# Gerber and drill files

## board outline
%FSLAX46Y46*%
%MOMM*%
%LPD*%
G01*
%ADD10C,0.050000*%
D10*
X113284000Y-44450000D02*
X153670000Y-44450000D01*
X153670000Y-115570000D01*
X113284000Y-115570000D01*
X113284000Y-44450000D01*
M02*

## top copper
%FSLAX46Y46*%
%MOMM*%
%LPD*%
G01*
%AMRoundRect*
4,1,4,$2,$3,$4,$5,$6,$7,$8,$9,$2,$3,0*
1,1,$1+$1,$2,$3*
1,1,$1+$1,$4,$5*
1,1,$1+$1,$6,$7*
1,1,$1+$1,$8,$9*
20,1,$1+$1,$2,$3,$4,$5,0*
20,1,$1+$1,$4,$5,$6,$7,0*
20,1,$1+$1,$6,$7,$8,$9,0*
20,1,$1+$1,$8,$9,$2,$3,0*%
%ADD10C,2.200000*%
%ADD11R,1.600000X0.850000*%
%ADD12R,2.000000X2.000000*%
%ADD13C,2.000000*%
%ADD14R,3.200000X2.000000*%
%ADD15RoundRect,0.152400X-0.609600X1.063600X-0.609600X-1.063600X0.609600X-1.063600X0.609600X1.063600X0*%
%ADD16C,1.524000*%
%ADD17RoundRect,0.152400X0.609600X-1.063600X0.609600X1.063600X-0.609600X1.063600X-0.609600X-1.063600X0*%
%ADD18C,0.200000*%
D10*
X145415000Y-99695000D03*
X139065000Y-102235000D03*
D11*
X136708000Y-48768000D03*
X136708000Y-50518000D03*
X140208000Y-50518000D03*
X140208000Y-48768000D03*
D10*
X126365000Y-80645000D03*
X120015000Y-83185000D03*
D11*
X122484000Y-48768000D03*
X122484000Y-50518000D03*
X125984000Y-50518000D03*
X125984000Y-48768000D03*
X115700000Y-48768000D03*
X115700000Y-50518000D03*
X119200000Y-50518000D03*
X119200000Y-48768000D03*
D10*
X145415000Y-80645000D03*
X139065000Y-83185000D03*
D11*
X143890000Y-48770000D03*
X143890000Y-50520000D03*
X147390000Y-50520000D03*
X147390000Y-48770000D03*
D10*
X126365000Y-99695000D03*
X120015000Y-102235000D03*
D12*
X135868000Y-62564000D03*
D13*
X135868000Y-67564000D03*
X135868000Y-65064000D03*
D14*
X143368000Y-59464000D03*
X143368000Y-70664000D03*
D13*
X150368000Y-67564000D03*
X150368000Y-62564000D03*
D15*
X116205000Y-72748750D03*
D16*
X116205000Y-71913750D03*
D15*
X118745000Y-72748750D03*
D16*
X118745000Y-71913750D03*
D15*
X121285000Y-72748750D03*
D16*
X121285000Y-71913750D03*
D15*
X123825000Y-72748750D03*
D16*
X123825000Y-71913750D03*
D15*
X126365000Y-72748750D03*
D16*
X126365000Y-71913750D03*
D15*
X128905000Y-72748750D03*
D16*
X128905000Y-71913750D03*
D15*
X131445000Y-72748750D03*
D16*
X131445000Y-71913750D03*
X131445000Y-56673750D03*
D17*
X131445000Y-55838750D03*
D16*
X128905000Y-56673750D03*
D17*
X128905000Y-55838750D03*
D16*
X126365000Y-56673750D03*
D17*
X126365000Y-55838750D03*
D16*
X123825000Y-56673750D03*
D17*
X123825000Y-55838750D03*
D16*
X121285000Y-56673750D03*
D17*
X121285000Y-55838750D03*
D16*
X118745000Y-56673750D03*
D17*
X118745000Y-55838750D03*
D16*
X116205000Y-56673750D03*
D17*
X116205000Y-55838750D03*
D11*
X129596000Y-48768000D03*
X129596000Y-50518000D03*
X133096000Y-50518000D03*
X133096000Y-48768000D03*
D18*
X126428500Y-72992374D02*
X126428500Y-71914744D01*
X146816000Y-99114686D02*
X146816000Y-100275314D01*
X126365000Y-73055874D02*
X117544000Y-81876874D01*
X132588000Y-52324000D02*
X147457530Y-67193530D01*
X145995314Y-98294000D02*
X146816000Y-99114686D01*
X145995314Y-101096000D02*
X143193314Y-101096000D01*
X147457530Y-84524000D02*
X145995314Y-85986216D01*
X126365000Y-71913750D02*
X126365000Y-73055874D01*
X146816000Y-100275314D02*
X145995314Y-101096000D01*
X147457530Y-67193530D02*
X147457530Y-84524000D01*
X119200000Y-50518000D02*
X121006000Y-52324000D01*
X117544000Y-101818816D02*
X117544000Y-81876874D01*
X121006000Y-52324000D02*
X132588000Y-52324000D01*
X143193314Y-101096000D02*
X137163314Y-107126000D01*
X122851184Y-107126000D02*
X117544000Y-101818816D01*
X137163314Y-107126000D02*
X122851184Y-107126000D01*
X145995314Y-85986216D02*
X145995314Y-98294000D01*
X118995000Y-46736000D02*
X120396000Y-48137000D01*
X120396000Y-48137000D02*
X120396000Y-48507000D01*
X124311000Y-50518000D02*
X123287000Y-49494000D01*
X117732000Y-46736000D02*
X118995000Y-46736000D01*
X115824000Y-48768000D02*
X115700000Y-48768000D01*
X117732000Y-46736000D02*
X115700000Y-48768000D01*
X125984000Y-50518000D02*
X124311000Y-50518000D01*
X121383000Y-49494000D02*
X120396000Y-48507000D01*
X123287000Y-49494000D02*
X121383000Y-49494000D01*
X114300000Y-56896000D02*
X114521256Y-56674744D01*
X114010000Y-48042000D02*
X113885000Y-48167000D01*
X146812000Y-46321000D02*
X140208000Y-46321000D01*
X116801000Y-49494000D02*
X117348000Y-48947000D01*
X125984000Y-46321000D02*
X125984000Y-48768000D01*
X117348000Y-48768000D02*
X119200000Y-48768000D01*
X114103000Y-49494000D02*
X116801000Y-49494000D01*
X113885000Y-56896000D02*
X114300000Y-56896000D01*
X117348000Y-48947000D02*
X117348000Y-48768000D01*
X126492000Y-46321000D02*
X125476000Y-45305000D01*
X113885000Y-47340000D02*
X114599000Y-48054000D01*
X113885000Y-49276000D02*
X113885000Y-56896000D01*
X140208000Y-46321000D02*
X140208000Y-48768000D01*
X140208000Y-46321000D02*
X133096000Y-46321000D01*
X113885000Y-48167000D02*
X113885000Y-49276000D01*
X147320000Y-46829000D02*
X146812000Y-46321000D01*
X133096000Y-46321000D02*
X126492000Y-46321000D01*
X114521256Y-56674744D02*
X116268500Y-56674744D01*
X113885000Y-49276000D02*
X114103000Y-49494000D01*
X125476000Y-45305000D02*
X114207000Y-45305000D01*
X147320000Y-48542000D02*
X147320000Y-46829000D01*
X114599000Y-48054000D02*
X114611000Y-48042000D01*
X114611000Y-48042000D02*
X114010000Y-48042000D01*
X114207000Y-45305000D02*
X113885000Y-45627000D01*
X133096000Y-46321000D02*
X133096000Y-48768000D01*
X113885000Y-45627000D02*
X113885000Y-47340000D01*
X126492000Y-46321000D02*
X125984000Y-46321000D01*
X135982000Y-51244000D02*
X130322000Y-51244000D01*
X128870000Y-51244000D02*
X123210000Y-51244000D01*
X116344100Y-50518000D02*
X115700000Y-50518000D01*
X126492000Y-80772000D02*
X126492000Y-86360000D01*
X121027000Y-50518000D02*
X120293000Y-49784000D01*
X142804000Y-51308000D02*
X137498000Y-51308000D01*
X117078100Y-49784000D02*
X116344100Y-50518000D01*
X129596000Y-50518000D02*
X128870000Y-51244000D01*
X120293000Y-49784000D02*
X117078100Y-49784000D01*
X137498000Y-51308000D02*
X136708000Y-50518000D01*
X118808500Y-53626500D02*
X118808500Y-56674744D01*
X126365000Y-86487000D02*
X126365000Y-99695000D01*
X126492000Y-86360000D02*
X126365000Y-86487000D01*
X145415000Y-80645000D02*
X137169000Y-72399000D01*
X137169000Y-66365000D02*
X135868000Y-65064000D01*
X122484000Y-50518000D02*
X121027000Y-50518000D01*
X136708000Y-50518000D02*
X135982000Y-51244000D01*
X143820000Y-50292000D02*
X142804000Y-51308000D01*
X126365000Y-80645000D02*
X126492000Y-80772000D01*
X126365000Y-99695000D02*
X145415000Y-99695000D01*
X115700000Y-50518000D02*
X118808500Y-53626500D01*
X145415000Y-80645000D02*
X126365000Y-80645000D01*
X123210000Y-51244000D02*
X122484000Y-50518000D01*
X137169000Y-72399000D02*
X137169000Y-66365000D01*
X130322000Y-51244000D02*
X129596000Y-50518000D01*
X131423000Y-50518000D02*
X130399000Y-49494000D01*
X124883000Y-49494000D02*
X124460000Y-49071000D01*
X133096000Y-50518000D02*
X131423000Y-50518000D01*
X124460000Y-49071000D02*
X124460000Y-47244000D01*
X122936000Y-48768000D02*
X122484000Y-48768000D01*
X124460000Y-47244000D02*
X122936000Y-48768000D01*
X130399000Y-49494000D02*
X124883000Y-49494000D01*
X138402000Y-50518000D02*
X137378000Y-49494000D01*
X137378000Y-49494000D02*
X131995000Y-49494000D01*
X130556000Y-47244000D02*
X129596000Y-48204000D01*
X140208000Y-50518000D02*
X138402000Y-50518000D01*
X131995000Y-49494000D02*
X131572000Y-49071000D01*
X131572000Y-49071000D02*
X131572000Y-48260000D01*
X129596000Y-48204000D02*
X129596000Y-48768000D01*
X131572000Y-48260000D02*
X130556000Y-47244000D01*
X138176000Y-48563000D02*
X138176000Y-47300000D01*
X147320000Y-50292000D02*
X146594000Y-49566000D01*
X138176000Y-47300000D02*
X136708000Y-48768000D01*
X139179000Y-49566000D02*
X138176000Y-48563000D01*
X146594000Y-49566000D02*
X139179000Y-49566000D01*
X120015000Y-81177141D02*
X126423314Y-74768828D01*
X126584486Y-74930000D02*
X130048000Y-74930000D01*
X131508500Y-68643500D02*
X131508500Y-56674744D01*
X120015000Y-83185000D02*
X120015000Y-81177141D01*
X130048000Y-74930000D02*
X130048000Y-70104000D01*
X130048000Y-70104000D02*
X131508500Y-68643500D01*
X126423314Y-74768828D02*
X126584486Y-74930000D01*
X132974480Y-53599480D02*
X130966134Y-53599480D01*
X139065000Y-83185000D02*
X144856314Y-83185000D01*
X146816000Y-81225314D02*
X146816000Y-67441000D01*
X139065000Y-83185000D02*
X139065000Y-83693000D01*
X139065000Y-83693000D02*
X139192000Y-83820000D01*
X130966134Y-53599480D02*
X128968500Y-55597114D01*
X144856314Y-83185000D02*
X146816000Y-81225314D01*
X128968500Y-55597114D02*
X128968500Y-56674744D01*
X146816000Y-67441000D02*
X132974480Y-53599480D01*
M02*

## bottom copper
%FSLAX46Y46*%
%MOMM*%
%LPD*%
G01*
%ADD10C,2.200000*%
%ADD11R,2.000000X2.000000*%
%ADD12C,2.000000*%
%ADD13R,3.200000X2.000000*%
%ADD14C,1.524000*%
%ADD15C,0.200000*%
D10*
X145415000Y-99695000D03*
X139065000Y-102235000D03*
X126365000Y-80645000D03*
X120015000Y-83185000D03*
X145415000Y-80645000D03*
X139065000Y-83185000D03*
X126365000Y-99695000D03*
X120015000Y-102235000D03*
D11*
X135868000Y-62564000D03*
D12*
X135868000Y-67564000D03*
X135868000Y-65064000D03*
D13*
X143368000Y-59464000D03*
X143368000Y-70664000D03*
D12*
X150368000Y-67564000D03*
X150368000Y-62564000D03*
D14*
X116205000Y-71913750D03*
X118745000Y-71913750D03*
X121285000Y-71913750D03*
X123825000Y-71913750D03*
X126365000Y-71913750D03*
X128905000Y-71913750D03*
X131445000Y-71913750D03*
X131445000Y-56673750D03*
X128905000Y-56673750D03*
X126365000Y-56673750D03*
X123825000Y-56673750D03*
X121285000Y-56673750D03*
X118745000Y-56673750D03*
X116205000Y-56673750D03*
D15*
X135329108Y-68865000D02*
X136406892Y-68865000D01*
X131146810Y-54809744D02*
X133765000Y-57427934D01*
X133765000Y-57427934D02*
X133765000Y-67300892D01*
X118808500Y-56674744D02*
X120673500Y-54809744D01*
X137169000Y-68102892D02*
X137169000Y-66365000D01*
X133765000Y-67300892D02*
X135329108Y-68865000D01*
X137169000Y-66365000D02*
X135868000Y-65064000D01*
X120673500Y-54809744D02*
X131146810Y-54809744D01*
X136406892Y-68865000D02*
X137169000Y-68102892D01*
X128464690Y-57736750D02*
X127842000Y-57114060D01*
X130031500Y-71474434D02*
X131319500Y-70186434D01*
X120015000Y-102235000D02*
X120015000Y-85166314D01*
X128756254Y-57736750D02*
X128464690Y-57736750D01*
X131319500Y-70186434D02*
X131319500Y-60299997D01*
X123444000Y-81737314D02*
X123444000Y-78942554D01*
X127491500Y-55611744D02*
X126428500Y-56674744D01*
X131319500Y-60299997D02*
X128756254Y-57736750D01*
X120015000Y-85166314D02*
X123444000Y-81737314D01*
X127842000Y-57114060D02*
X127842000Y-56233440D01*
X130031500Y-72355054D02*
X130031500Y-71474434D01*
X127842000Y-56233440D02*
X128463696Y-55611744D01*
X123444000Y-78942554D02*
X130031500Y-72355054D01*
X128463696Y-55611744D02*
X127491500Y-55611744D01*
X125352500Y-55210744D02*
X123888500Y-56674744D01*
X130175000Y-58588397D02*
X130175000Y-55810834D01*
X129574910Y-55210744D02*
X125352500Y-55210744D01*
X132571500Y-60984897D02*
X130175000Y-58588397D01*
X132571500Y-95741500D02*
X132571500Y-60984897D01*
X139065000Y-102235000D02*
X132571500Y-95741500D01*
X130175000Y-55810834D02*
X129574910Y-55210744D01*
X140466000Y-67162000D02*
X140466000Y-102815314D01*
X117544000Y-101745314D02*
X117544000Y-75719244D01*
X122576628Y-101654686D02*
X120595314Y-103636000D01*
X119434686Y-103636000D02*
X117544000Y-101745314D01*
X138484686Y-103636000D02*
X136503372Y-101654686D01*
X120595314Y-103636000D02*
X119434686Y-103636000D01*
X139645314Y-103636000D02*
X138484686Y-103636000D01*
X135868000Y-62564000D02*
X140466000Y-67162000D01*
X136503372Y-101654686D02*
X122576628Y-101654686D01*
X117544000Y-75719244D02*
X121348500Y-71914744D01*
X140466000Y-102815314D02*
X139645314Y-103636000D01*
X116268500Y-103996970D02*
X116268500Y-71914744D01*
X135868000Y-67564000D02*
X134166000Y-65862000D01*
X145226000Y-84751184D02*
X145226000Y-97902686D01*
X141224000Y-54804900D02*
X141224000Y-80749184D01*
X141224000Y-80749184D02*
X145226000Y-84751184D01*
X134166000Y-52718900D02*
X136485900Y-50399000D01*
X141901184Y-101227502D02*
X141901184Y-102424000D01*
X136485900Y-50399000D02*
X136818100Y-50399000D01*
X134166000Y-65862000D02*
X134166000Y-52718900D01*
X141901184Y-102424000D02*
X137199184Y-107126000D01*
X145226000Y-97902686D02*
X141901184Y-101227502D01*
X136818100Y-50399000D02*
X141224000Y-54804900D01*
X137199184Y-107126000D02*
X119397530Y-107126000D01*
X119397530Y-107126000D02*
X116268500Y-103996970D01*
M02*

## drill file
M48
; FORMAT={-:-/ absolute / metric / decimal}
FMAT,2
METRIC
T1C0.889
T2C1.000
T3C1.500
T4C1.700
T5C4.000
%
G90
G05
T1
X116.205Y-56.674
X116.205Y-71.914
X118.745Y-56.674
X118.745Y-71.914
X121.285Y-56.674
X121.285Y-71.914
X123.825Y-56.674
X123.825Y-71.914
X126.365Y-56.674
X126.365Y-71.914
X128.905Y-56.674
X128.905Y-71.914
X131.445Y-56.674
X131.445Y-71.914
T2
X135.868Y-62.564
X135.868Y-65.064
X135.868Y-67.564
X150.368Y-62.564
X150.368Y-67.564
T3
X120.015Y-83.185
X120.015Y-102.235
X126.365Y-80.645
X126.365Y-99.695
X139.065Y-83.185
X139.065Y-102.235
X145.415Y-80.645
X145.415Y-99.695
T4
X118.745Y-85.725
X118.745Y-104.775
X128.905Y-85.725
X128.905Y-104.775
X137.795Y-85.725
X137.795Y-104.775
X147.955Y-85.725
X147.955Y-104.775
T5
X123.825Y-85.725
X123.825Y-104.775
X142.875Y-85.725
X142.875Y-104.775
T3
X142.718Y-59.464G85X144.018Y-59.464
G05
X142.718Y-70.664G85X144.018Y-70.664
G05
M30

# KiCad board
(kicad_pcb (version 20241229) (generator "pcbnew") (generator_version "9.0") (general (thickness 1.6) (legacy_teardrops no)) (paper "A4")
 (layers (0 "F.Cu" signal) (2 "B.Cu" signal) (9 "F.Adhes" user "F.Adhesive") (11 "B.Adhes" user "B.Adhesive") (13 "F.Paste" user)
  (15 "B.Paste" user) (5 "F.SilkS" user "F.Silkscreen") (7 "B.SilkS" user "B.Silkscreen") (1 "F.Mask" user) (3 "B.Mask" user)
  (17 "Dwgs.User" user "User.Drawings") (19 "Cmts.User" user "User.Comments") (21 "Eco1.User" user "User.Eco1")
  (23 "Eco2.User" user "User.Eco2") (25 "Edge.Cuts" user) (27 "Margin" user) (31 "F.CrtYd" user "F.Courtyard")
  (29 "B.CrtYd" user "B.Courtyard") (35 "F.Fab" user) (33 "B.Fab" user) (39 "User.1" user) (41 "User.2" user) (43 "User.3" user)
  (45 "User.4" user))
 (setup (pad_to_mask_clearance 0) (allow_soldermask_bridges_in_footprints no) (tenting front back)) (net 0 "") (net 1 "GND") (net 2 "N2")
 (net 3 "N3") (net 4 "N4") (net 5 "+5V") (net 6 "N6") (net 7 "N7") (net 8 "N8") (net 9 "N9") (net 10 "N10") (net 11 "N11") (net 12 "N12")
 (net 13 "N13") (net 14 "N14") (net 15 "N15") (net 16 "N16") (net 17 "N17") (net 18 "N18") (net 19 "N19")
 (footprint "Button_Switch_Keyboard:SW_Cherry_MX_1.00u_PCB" (layer "F.Cu") (at 145.415 99.695)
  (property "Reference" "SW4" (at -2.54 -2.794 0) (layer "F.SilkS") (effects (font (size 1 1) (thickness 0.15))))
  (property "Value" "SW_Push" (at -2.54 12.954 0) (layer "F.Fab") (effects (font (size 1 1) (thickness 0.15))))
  (pad "" np_thru_hole circle (at -7.62 5.08) (size 1.7 1.7) (drill 1.7) (layers "*.Cu" "*.Mask"))
  (pad "" np_thru_hole circle (at -2.54 5.08) (size 4 4) (drill 4) (layers "*.Cu" "*.Mask"))
  (pad "" np_thru_hole circle (at 2.54 5.08) (size 1.7 1.7) (drill 1.7) (layers "*.Cu" "*.Mask"))
  (pad "1" thru_hole circle (at 0 0) (size 2.2 2.2) (drill 1.5) (layers "*.Cu" "*.Mask") (remove_unused_layers no) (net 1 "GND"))
  (pad "2" thru_hole circle (at -6.35 2.54) (size 2.2 2.2) (drill 1.5) (layers "*.Cu" "*.Mask") (remove_unused_layers no) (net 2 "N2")))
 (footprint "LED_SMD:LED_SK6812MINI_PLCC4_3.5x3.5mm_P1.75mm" (layer "F.Cu") (at 138.458 49.643)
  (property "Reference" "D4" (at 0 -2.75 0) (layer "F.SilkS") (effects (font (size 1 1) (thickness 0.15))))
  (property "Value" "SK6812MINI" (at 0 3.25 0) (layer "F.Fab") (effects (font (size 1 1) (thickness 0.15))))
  (pad "1" smd rect (at -1.75 -0.875) (size 1.6 0.85) (layers "F.Cu" "F.Mask" "F.Paste") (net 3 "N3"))
  (pad "2" smd rect (at -1.75 0.875) (size 1.6 0.85) (layers "F.Cu" "F.Mask" "F.Paste") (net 1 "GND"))
  (pad "3" smd rect (at 1.75 0.875) (size 1.6 0.85) (layers "F.Cu" "F.Mask" "F.Paste") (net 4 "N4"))
  (pad "4" smd rect (at 1.75 -0.875) (size 1.6 0.85) (layers "F.Cu" "F.Mask" "F.Paste") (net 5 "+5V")))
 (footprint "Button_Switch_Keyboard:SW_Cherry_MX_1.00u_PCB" (layer "F.Cu") (at 126.365 80.645)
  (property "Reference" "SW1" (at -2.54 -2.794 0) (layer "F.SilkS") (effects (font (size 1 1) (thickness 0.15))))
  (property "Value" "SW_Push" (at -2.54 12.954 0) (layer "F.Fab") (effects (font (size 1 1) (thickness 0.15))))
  (pad "" np_thru_hole circle (at -7.62 5.08) (size 1.7 1.7) (drill 1.7) (layers "*.Cu" "*.Mask"))
  (pad "" np_thru_hole circle (at -2.54 5.08) (size 4 4) (drill 4) (layers "*.Cu" "*.Mask"))
  (pad "" np_thru_hole circle (at 2.54 5.08) (size 1.7 1.7) (drill 1.7) (layers "*.Cu" "*.Mask"))
  (pad "1" thru_hole circle (at 0 0) (size 2.2 2.2) (drill 1.5) (layers "*.Cu" "*.Mask") (remove_unused_layers no) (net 1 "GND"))
  (pad "2" thru_hole circle (at -6.35 2.54) (size 2.2 2.2) (drill 1.5) (layers "*.Cu" "*.Mask") (remove_unused_layers no) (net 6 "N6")))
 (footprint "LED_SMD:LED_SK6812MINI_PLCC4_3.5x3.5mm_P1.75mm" (layer "F.Cu") (at 124.234 49.643)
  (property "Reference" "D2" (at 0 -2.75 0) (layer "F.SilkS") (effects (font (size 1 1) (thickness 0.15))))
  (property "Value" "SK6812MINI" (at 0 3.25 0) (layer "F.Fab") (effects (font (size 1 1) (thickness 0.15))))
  (pad "1" smd rect (at -1.75 -0.875) (size 1.6 0.85) (layers "F.Cu" "F.Mask" "F.Paste") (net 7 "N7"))
  (pad "2" smd rect (at -1.75 0.875) (size 1.6 0.85) (layers "F.Cu" "F.Mask" "F.Paste") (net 1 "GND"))
  (pad "3" smd rect (at 1.75 0.875) (size 1.6 0.85) (layers "F.Cu" "F.Mask" "F.Paste") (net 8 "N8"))
  (pad "4" smd rect (at 1.75 -0.875) (size 1.6 0.85) (layers "F.Cu" "F.Mask" "F.Paste") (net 5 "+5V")))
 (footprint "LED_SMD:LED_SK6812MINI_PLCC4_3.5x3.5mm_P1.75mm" (layer "F.Cu") (at 117.45 49.643)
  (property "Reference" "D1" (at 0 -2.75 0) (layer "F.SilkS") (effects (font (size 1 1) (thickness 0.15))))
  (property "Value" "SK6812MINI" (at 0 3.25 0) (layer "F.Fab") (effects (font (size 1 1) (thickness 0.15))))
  (pad "1" smd rect (at -1.75 -0.875) (size 1.6 0.85) (layers "F.Cu" "F.Mask" "F.Paste") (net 8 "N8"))
  (pad "2" smd rect (at -1.75 0.875) (size 1.6 0.85) (layers "F.Cu" "F.Mask" "F.Paste") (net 1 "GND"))
  (pad "3" smd rect (at 1.75 0.875) (size 1.6 0.85) (layers "F.Cu" "F.Mask" "F.Paste") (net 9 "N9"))
  (pad "4" smd rect (at 1.75 -0.875) (size 1.6 0.85) (layers "F.Cu" "F.Mask" "F.Paste") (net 5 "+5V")))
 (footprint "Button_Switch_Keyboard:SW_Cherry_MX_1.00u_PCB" (layer "F.Cu") (at 145.415 80.645)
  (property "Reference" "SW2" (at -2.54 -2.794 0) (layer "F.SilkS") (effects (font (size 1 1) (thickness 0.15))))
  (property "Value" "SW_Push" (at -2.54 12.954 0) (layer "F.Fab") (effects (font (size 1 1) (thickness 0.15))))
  (pad "" np_thru_hole circle (at -7.62 5.08) (size 1.7 1.7) (drill 1.7) (layers "*.Cu" "*.Mask"))
  (pad "" np_thru_hole circle (at -2.54 5.08) (size 4 4) (drill 4) (layers "*.Cu" "*.Mask"))
  (pad "" np_thru_hole circle (at 2.54 5.08) (size 1.7 1.7) (drill 1.7) (layers "*.Cu" "*.Mask"))
  (pad "1" thru_hole circle (at 0 0) (size 2.2 2.2) (drill 1.5) (layers "*.Cu" "*.Mask") (remove_unused_layers no) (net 1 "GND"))
  (pad "2" thru_hole circle (at -6.35 2.54) (size 2.2 2.2) (drill 1.5) (layers "*.Cu" "*.Mask") (remove_unused_layers no) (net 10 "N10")))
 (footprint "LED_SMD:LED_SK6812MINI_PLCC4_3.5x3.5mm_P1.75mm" (layer "F.Cu") (at 145.64 49.645)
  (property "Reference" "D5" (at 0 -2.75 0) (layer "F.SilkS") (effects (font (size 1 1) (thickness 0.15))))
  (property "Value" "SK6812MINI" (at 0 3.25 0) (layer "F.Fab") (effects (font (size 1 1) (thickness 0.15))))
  (pad "1" smd rect (at -1.75 -0.875) (size 1.6 0.85) (layers "F.Cu" "F.Mask" "F.Paste") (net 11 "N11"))
  (pad "2" smd rect (at -1.75 0.875) (size 1.6 0.85) (layers "F.Cu" "F.Mask" "F.Paste") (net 1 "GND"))
  (pad "3" smd rect (at 1.75 0.875) (size 1.6 0.85) (layers "F.Cu" "F.Mask" "F.Paste") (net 3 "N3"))
  (pad "4" smd rect (at 1.75 -0.875) (size 1.6 0.85) (layers "F.Cu" "F.Mask" "F.Paste") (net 5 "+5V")))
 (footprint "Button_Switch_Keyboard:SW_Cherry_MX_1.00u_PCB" (layer "F.Cu") (at 126.365 99.695)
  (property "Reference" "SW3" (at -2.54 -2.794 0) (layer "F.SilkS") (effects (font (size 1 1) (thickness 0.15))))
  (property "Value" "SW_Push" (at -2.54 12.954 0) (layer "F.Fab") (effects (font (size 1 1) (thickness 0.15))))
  (pad "" np_thru_hole circle (at -7.62 5.08) (size 1.7 1.7) (drill 1.7) (layers "*.Cu" "*.Mask"))
  (pad "" np_thru_hole circle (at -2.54 5.08) (size 4 4) (drill 4) (layers "*.Cu" "*.Mask"))
  (pad "" np_thru_hole circle (at 2.54 5.08) (size 1.7 1.7) (drill 1.7) (layers "*.Cu" "*.Mask"))
  (pad "1" thru_hole circle (at 0 0) (size 2.2 2.2) (drill 1.5) (layers "*.Cu" "*.Mask") (remove_unused_layers no) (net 1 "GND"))
  (pad "2" thru_hole circle (at -6.35 2.54) (size 2.2 2.2) (drill 1.5) (layers "*.Cu" "*.Mask") (remove_unused_layers no) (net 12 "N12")))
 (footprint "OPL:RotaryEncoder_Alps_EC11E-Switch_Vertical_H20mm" (layer "F.Cu") (at 135.868 62.564)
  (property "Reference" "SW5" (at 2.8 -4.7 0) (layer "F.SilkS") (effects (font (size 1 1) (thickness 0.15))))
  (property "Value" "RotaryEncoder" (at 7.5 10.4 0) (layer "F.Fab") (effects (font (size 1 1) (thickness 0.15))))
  (pad "A" thru_hole rect (at 0 0) (size 2 2) (drill 1) (layers "*.Cu" "*.Mask") (remove_unused_layers no) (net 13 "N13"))
  (pad "B" thru_hole circle (at 0 5) (size 2 2) (drill 1) (layers "*.Cu" "*.Mask") (remove_unused_layers no) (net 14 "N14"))
  (pad "C" thru_hole circle (at 0 2.5) (size 2 2) (drill 1) (layers "*.Cu" "*.Mask") (remove_unused_layers no) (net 1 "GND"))
  (pad "MP" thru_hole rect (at 7.5 -3.1) (size 3.2 2) (drill oval 2.8 1.5) (layers "*.Cu" "*.Mask") (remove_unused_layers no))
  (pad "MP" thru_hole rect (at 7.5 8.1) (size 3.2 2) (drill oval 2.8 1.5) (layers "*.Cu" "*.Mask") (remove_unused_layers no))
  (pad "S1" thru_hole circle (at 14.5 5) (size 2 2) (drill 1) (layers "*.Cu" "*.Mask") (remove_unused_layers no))
  (pad "S2" thru_hole circle (at 14.5 0) (size 2 2) (drill 1) (layers "*.Cu" "*.Mask") (remove_unused_layers no)))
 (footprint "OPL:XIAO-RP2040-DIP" (layer "F.Cu") (at 123.825 64.29375 90)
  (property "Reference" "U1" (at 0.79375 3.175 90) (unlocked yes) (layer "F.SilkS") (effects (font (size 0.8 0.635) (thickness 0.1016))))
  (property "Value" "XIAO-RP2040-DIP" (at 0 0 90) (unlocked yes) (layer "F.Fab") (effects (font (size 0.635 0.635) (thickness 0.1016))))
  (pad "1" smd roundrect (at -8.455 -7.62 270) (size 2.432 1.524) (layers "F.Cu" "F.Mask") (roundrect_rratio 0.1) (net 14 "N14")
   (thermal_bridge_angle 45))
  (pad "1" thru_hole circle (at -7.62 -7.62 270) (size 1.524 1.524) (drill 0.889) (layers "*.Cu" "*.Mask") (remove_unused_layers no)
   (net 14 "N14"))
  (pad "2" smd roundrect (at -8.455 -5.08 270) (size 2.432 1.524) (layers "F.Cu" "F.Mask") (roundrect_rratio 0.1) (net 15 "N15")
   (thermal_bridge_angle 45))
  (pad "2" thru_hole circle (at -7.62 -5.08 270) (size 1.524 1.524) (drill 0.889) (layers "*.Cu" "*.Mask") (remove_unused_layers no)
   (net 15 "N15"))
  (pad "3" smd roundrect (at -8.455 -2.54 270) (size 2.432 1.524) (layers "F.Cu" "F.Mask") (roundrect_rratio 0.1) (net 13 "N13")
   (thermal_bridge_angle 45))
  (pad "3" thru_hole circle (at -7.62 -2.54 270) (size 1.524 1.524) (drill 0.889) (layers "*.Cu" "*.Mask") (remove_unused_layers no)
   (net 13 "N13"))
  (pad "4" smd roundrect (at -8.455 0 270) (size 2.432 1.524) (layers "F.Cu" "F.Mask") (roundrect_rratio 0.1) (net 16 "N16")
   (thermal_bridge_angle 45))
  (pad "4" thru_hole circle (at -7.62 0 270) (size 1.524 1.524) (drill 0.889) (layers "*.Cu" "*.Mask") (remove_unused_layers no)
   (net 16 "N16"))
  (pad "5" smd roundrect (at -8.455 2.54 270) (size 2.432 1.524) (layers "F.Cu" "F.Mask") (roundrect_rratio 0.1) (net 9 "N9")
   (thermal_bridge_angle 45))
  (pad "5" thru_hole circle (at -7.62 2.54 270) (size 1.524 1.524) (drill 0.889) (layers "*.Cu" "*.Mask") (remove_unused_layers no)
   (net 9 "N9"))
  (pad "6" smd roundrect (at -8.455 5.08 270) (size 2.432 1.524) (layers "F.Cu" "F.Mask") (roundrect_rratio 0.1) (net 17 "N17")
   (thermal_bridge_angle 45))
  (pad "6" thru_hole circle (at -7.62 5.08 270) (size 1.524 1.524) (drill 0.889) (layers "*.Cu" "*.Mask") (remove_unused_layers no)
   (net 17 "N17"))
  (pad "7" smd roundrect (at -8.455 7.62 270) (size 2.432 1.524) (layers "F.Cu" "F.Mask") (roundrect_rratio 0.1) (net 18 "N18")
   (thermal_bridge_angle 45))
  (pad "7" thru_hole circle (at -7.62 7.62 270) (size 1.524 1.524) (drill 0.889) (layers "*.Cu" "*.Mask") (remove_unused_layers no)
   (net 18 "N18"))
  (pad "8" thru_hole circle (at 7.62 7.62 90) (size 1.524 1.524) (drill 0.889) (layers "*.Cu" "*.Mask") (remove_unused_layers no)
   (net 6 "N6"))
  (pad "8" smd roundrect (at 8.455 7.62 90) (size 2.432 1.524) (layers "F.Cu" "F.Mask") (roundrect_rratio 0.1) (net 6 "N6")
   (thermal_bridge_angle 45))
  (pad "9" thru_hole circle (at 7.62 5.08 90) (size 1.524 1.524) (drill 0.889) (layers "*.Cu" "*.Mask") (remove_unused_layers no)
   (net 10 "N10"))
  (pad "9" smd roundrect (at 8.455 5.08 90) (size 2.432 1.524) (layers "F.Cu" "F.Mask") (roundrect_rratio 0.1) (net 10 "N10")
   (thermal_bridge_angle 45))
  (pad "10" thru_hole circle (at 7.62 2.54 90) (size 1.524 1.524) (drill 0.889) (layers "*.Cu" "*.Mask") (remove_unused_layers no)
   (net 12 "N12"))
  (pad "10" smd roundrect (at 8.455 2.54 90) (size 2.432 1.524) (layers "F.Cu" "F.Mask") (roundrect_rratio 0.1) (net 12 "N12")
   (thermal_bridge_angle 45))
  (pad "11" thru_hole circle (at 7.62 0 90) (size 1.524 1.524) (drill 0.889) (layers "*.Cu" "*.Mask") (remove_unused_layers no) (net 2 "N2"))
  (pad "11" smd roundrect (at 8.455 0 90) (size 2.432 1.524) (layers "F.Cu" "F.Mask") (roundrect_rratio 0.1) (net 2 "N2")
   (thermal_bridge_angle 45))
  (pad "12" thru_hole circle (at 7.62 -2.54 90) (size 1.524 1.524) (drill 0.889) (layers "*.Cu" "*.Mask") (remove_unused_layers no)
   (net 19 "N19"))
  (pad "12" smd roundrect (at 8.455 -2.54 90) (size 2.432 1.524) (layers "F.Cu" "F.Mask") (roundrect_rratio 0.1) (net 19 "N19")
   (thermal_bridge_angle 45))
  (pad "13" thru_hole circle (at 7.62 -5.08 90) (size 1.524 1.524) (drill 0.889) (layers "*.Cu" "*.Mask") (remove_unused_layers no)
   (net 1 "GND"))
  (pad "13" smd roundrect (at 8.455 -5.08 90) (size 2.432 1.524) (layers "F.Cu" "F.Mask") (roundrect_rratio 0.1) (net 1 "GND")
   (thermal_bridge_angle 45))
  (pad "14" thru_hole circle (at 7.62 -7.62 90) (size 1.524 1.524) (drill 0.889) (layers "*.Cu" "*.Mask") (remove_unused_layers no)
   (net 5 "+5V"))
  (pad "14" smd roundrect (at 8.455 -7.62 90) (size 2.432 1.524) (layers "F.Cu" "F.Mask") (roundrect_rratio 0.1) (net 5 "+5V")
   (thermal_bridge_angle 45)))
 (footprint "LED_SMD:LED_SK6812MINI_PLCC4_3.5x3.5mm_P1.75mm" (layer "F.Cu") (at 131.346 49.643)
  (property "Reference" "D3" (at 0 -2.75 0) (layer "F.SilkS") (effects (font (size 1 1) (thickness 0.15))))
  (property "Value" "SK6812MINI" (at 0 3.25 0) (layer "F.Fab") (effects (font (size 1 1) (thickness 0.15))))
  (pad "1" smd rect (at -1.75 -0.875) (size 1.6 0.85) (layers "F.Cu" "F.Mask" "F.Paste") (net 4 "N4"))
  (pad "2" smd rect (at -1.75 0.875) (size 1.6 0.85) (layers "F.Cu" "F.Mask" "F.Paste") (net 1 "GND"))
  (pad "3" smd rect (at 1.75 0.875) (size 1.6 0.85) (layers "F.Cu" "F.Mask" "F.Paste") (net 7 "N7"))
  (pad "4" smd rect (at 1.75 -0.875) (size 1.6 0.85) (layers "F.Cu" "F.Mask" "F.Paste") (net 5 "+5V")))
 (gr_rect (start 113.284 44.45) (end 153.67 115.57) (stroke (width 0.05) (type default)) (fill no) (layer "Edge.Cuts"))
 (segment (start 126.4285 72.992374) (end 126.4285 71.914744) (width 0.2) (layer "F.Cu") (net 9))
 (segment (start 146.816 99.114686) (end 146.816 100.275314) (width 0.2) (layer "F.Cu") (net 9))
 (segment (start 126.365 73.055874) (end 117.544 81.876874) (width 0.2) (layer "F.Cu") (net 9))
 (segment (start 132.588 52.324) (end 147.45753 67.19353) (width 0.2) (layer "F.Cu") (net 9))
 (segment (start 145.995314 98.294) (end 146.816 99.114686) (width 0.2) (layer "F.Cu") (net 9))
 (segment (start 145.995314 101.096) (end 143.193314 101.096) (width 0.2) (layer "F.Cu") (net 9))
 (segment (start 147.45753 84.524) (end 145.995314 85.986216) (width 0.2) (layer "F.Cu") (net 9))
 (segment (start 126.365 71.91375) (end 126.365 73.055874) (width 0.2) (layer "F.Cu") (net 9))
 (segment (start 146.816 100.275314) (end 145.995314 101.096) (width 0.2) (layer "F.Cu") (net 9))
 (segment (start 147.45753 67.19353) (end 147.45753 84.524) (width 0.2) (layer "F.Cu") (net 9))
 (segment (start 119.2 50.518) (end 121.006 52.324) (width 0.2) (layer "F.Cu") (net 9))
 (segment (start 117.544 101.818816) (end 117.544 81.876874) (width 0.2) (layer "F.Cu") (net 9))
 (segment (start 121.006 52.324) (end 132.588 52.324) (width 0.2) (layer "F.Cu") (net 9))
 (segment (start 143.193314 101.096) (end 137.163314 107.126) (width 0.2) (layer "F.Cu") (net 9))
 (segment (start 122.851184 107.126) (end 117.544 101.818816) (width 0.2) (layer "F.Cu") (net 9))
 (segment (start 137.163314 107.126) (end 122.851184 107.126) (width 0.2) (layer "F.Cu") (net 9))
 (segment (start 145.995314 85.986216) (end 145.995314 98.294) (width 0.2) (layer "F.Cu") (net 9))
 (segment (start 118.995 46.736) (end 120.396 48.137) (width 0.2) (layer "F.Cu") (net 8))
 (segment (start 120.396 48.137) (end 120.396 48.507) (width 0.2) (layer "F.Cu") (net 8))
 (segment (start 124.311 50.518) (end 123.287 49.494) (width 0.2) (layer "F.Cu") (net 8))
 (segment (start 117.732 46.736) (end 118.995 46.736) (width 0.2) (layer "F.Cu") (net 8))
 (segment (start 115.824 48.768) (end 115.7 48.768) (width 0.2) (layer "F.Cu") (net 8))
 (segment (start 117.732 46.736) (end 115.7 48.768) (width 0.2) (layer "F.Cu") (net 8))
 (segment (start 125.984 50.518) (end 124.311 50.518) (width 0.2) (layer "F.Cu") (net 8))
 (segment (start 121.383 49.494) (end 120.396 48.507) (width 0.2) (layer "F.Cu") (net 8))
 (segment (start 123.287 49.494) (end 121.383 49.494) (width 0.2) (layer "F.Cu") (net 8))
 (segment (start 114.3 56.896) (end 114.521256 56.674744) (width 0.2) (layer "F.Cu") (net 5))
 (segment (start 114.01 48.042) (end 113.885 48.167) (width 0.2) (layer "F.Cu") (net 5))
 (segment (start 146.812 46.321) (end 140.208 46.321) (width 0.2) (layer "F.Cu") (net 5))
 (segment (start 116.801 49.494) (end 117.348 48.947) (width 0.2) (layer "F.Cu") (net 5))
 (segment (start 125.984 46.321) (end 125.984 48.768) (width 0.2) (layer "F.Cu") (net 5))
 (segment (start 117.348 48.768) (end 119.2 48.768) (width 0.2) (layer "F.Cu") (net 5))
 (segment (start 114.103 49.494) (end 116.801 49.494) (width 0.2) (layer "F.Cu") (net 5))
 (segment (start 113.885 56.896) (end 114.3 56.896) (width 0.2) (layer "F.Cu") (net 5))
 (segment (start 117.348 48.947) (end 117.348 48.768) (width 0.2) (layer "F.Cu") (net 5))
 (segment (start 126.492 46.321) (end 125.476 45.305) (width 0.2) (layer "F.Cu") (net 5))
 (segment (start 113.885 47.34) (end 114.599 48.054) (width 0.2) (layer "F.Cu") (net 5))
 (segment (start 113.885 49.276) (end 113.885 56.896) (width 0.2) (layer "F.Cu") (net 5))
 (segment (start 140.208 46.321) (end 140.208 48.768) (width 0.2) (layer "F.Cu") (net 5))
 (segment (start 140.208 46.321) (end 133.096 46.321) (width 0.2) (layer "F.Cu") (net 5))
 (segment (start 113.885 48.167) (end 113.885 49.276) (width 0.2) (layer "F.Cu") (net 5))
 (segment (start 147.32 46.829) (end 146.812 46.321) (width 0.2) (layer "F.Cu") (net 5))
 (segment (start 133.096 46.321) (end 126.492 46.321) (width 0.2) (layer "F.Cu") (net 5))
 (segment (start 114.521256 56.674744) (end 116.2685 56.674744) (width 0.2) (layer "F.Cu") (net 5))
 (segment (start 113.885 49.276) (end 114.103 49.494) (width 0.2) (layer "F.Cu") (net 5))
 (segment (start 125.476 45.305) (end 114.207 45.305) (width 0.2) (layer "F.Cu") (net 5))
 (segment (start 147.32 48.542) (end 147.32 46.829) (width 0.2) (layer "F.Cu") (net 5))
 (segment (start 114.599 48.054) (end 114.611 48.042) (width 0.2) (layer "F.Cu") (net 5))
 (segment (start 114.611 48.042) (end 114.01 48.042) (width 0.2) (layer "F.Cu") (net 5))
 (segment (start 114.207 45.305) (end 113.885 45.627) (width 0.2) (layer "F.Cu") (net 5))
 (segment (start 133.096 46.321) (end 133.096 48.768) (width 0.2) (layer "F.Cu") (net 5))
 (segment (start 113.885 45.627) (end 113.885 47.34) (width 0.2) (layer "F.Cu") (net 5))
 (segment (start 126.492 46.321) (end 125.984 46.321) (width 0.2) (layer "F.Cu") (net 5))
 (segment (start 135.982 51.244) (end 130.322 51.244) (width 0.2) (layer "F.Cu") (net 1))
 (segment (start 128.87 51.244) (end 123.21 51.244) (width 0.2) (layer "F.Cu") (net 1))
 (segment (start 116.3441 50.518) (end 115.7 50.518) (width 0.2) (layer "F.Cu") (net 1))
 (segment (start 126.492 80.772) (end 126.492 86.36) (width 0.2) (layer "F.Cu") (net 1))
 (segment (start 121.027 50.518) (end 120.293 49.784) (width 0.2) (layer "F.Cu") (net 1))
 (segment (start 142.804 51.308) (end 137.498 51.308) (width 0.2) (layer "F.Cu") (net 1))
 (segment (start 117.0781 49.784) (end 116.3441 50.518) (width 0.2) (layer "F.Cu") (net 1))
 (segment (start 129.596 50.518) (end 128.87 51.244) (width 0.2) (layer "F.Cu") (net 1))
 (segment (start 120.293 49.784) (end 117.0781 49.784) (width 0.2) (layer "F.Cu") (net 1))
 (segment (start 137.498 51.308) (end 136.708 50.518) (width 0.2) (layer "F.Cu") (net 1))
 (segment (start 118.8085 53.6265) (end 118.8085 56.674744) (width 0.2) (layer "F.Cu") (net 1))
 (segment (start 126.365 86.487) (end 126.365 99.695) (width 0.2) (layer "F.Cu") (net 1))
 (segment (start 126.492 86.36) (end 126.365 86.487) (width 0.2) (layer "F.Cu") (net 1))
 (segment (start 145.415 80.645) (end 137.169 72.399) (width 0.2) (layer "F.Cu") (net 1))
 (segment (start 137.169 66.365) (end 135.868 65.064) (width 0.2) (layer "F.Cu") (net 1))
 (segment (start 122.484 50.518) (end 121.027 50.518) (width 0.2) (layer "F.Cu") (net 1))
 (segment (start 136.708 50.518) (end 135.982 51.244) (width 0.2) (layer "F.Cu") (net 1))
 (segment (start 143.82 50.292) (end 142.804 51.308) (width 0.2) (layer "F.Cu") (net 1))
 (segment (start 126.365 80.645) (end 126.492 80.772) (width 0.2) (layer "F.Cu") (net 1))
 (segment (start 126.365 99.695) (end 145.415 99.695) (width 0.2) (layer "F.Cu") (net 1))
 (segment (start 115.7 50.518) (end 118.8085 53.6265) (width 0.2) (layer "F.Cu") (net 1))
 (segment (start 145.415 80.645) (end 126.365 80.645) (width 0.2) (layer "F.Cu") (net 1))
 (segment (start 123.21 51.244) (end 122.484 50.518) (width 0.2) (layer "F.Cu") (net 1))
 (segment (start 137.169 72.399) (end 137.169 66.365) (width 0.2) (layer "F.Cu") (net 1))
 (segment (start 130.322 51.244) (end 129.596 50.518) (width 0.2) (layer "F.Cu") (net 1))
 (segment (start 135.329108 68.865) (end 136.406892 68.865) (width 0.2) (layer "B.Cu") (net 1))
 (segment (start 131.14681 54.809744) (end 133.765 57.427934) (width 0.2) (layer "B.Cu") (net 1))
 (segment (start 133.765 57.427934) (end 133.765 67.300892) (width 0.2) (layer "B.Cu") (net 1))
 (segment (start 118.8085 56.674744) (end 120.6735 54.809744) (width 0.2) (layer "B.Cu") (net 1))
 (segment (start 137.169 68.102892) (end 137.169 66.365) (width 0.2) (layer "B.Cu") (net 1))
 (segment (start 133.765 67.300892) (end 135.329108 68.865) (width 0.2) (layer "B.Cu") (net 1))
 (segment (start 137.169 66.365) (end 135.868 65.064) (width 0.2) (layer "B.Cu") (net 1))
 (segment (start 120.6735 54.809744) (end 131.14681 54.809744) (width 0.2) (layer "B.Cu") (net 1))
 (segment (start 136.406892 68.865) (end 137.169 68.102892) (width 0.2) (layer "B.Cu") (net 1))
 (segment (start 131.423 50.518) (end 130.399 49.494) (width 0.2) (layer "F.Cu") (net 7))
 (segment (start 124.883 49.494) (end 124.46 49.071) (width 0.2) (layer "F.Cu") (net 7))
 (segment (start 133.096 50.518) (end 131.423 50.518) (width 0.2) (layer "F.Cu") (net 7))
 (segment (start 124.46 49.071) (end 124.46 47.244) (width 0.2) (layer "F.Cu") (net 7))
 (segment (start 122.936 48.768) (end 122.484 48.768) (width 0.2) (layer "F.Cu") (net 7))
 (segment (start 124.46 47.244) (end 122.936 48.768) (width 0.2) (layer "F.Cu") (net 7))
 (segment (start 130.399 49.494) (end 124.883 49.494) (width 0.2) (layer "F.Cu") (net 7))
 (segment (start 138.402 50.518) (end 137.378 49.494) (width 0.2) (layer "F.Cu") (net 4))
 (segment (start 137.378 49.494) (end 131.995 49.494) (width 0.2) (layer "F.Cu") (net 4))
 (segment (start 130.556 47.244) (end 129.596 48.204) (width 0.2) (layer "F.Cu") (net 4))
 (segment (start 140.208 50.518) (end 138.402 50.518) (width 0.2) (layer "F.Cu") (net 4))
 (segment (start 131.995 49.494) (end 131.572 49.071) (width 0.2) (layer "F.Cu") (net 4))
 (segment (start 131.572 49.071) (end 131.572 48.26) (width 0.2) (layer "F.Cu") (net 4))
 (segment (start 129.596 48.204) (end 129.596 48.768) (width 0.2) (layer "F.Cu") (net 4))
 (segment (start 131.572 48.26) (end 130.556 47.244) (width 0.2) (layer "F.Cu") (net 4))
 (segment (start 138.176 48.563) (end 138.176 47.3) (width 0.2) (layer "F.Cu") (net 3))
 (segment (start 147.32 50.292) (end 146.594 49.566) (width 0.2) (layer "F.Cu") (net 3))
 (segment (start 138.176 47.3) (end 136.708 48.768) (width 0.2) (layer "F.Cu") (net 3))
 (segment (start 139.179 49.566) (end 138.176 48.563) (width 0.2) (layer "F.Cu") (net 3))
 (segment (start 146.594 49.566) (end 139.179 49.566) (width 0.2) (layer "F.Cu") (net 3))
 (segment (start 120.015 81.177141) (end 126.423314 74.768828) (width 0.2) (layer "F.Cu") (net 6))
 (segment (start 126.584486 74.93) (end 130.048 74.93) (width 0.2) (layer "F.Cu") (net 6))
 (segment (start 131.5085 68.6435) (end 131.5085 56.674744) (width 0.2) (layer "F.Cu") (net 6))
 (segment (start 120.015 83.185) (end 120.015 81.177141) (width 0.2) (layer "F.Cu") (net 6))
 (segment (start 130.048 74.93) (end 130.048 70.104) (width 0.2) (layer "F.Cu") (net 6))
 (segment (start 130.048 70.104) (end 131.5085 68.6435) (width 0.2) (layer "F.Cu") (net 6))
 (segment (start 126.423314 74.768828) (end 126.584486 74.93) (width 0.2) (layer "F.Cu") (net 6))
 (segment (start 132.97448 53.59948) (end 130.966134 53.59948) (width 0.2) (layer "F.Cu") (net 10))
 (segment (start 139.065 83.185) (end 144.856314 83.185) (width 0.2) (layer "F.Cu") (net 10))
 (segment (start 146.816 81.225314) (end 146.816 67.441) (width 0.2) (layer "F.Cu") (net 10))
 (segment (start 139.065 83.185) (end 139.065 83.693) (width 0.2) (layer "F.Cu") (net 10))
 (segment (start 139.065 83.693) (end 139.192 83.82) (width 0.2) (layer "F.Cu") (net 10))
 (segment (start 130.966134 53.59948) (end 128.9685 55.597114) (width 0.2) (layer "F.Cu") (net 10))
 (segment (start 144.856314 83.185) (end 146.816 81.225314) (width 0.2) (layer "F.Cu") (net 10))
 (segment (start 128.9685 55.597114) (end 128.9685 56.674744) (width 0.2) (layer "F.Cu") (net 10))
 (segment (start 146.816 67.441) (end 132.97448 53.59948) (width 0.2) (layer "F.Cu") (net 10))
 (segment (start 128.46469 57.73675) (end 127.842 57.11406) (width 0.2) (layer "B.Cu") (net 12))
 (segment (start 130.0315 71.474434) (end 131.3195 70.186434) (width 0.2) (layer "B.Cu") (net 12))
 (segment (start 120.015 102.235) (end 120.015 85.166314) (width 0.2) (layer "B.Cu") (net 12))
 (segment (start 128.756254 57.73675) (end 128.46469 57.73675) (width 0.2) (layer "B.Cu") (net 12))
 (segment (start 131.3195 70.186434) (end 131.3195 60.299997) (width 0.2) (layer "B.Cu") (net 12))
 (segment (start 123.444 81.737314) (end 123.444 78.942554) (width 0.2) (layer "B.Cu") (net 12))
 (segment (start 127.4915 55.611744) (end 126.4285 56.674744) (width 0.2) (layer "B.Cu") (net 12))
 (segment (start 131.3195 60.299997) (end 128.756254 57.73675) (width 0.2) (layer "B.Cu") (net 12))
 (segment (start 120.015 85.166314) (end 123.444 81.737314) (width 0.2) (layer "B.Cu") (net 12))
 (segment (start 127.842 57.11406) (end 127.842 56.23344) (width 0.2) (layer "B.Cu") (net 12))
 (segment (start 130.0315 72.355054) (end 130.0315 71.474434) (width 0.2) (layer "B.Cu") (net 12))
 (segment (start 127.842 56.23344) (end 128.463696 55.611744) (width 0.2) (layer "B.Cu") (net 12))
 (segment (start 123.444 78.942554) (end 130.0315 72.355054) (width 0.2) (layer "B.Cu") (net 12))
 (segment (start 128.463696 55.611744) (end 127.4915 55.611744) (width 0.2) (layer "B.Cu") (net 12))
 (segment (start 125.3525 55.210744) (end 123.8885 56.674744) (width 0.2) (layer "B.Cu") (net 2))
 (segment (start 130.175 58.588397) (end 130.175 55.810834) (width 0.2) (layer "B.Cu") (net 2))
 (segment (start 129.57491 55.210744) (end 125.3525 55.210744) (width 0.2) (layer "B.Cu") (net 2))
 (segment (start 132.5715 60.984897) (end 130.175 58.588397) (width 0.2) (layer "B.Cu") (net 2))
 (segment (start 132.5715 95.7415) (end 132.5715 60.984897) (width 0.2) (layer "B.Cu") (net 2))
 (segment (start 139.065 102.235) (end 132.5715 95.7415) (width 0.2) (layer "B.Cu") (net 2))
 (segment (start 130.175 55.810834) (end 129.57491 55.210744) (width 0.2) (layer "B.Cu") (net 2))
 (segment (start 140.466 67.162) (end 140.466 102.815314) (width 0.2) (layer "B.Cu") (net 13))
 (segment (start 117.544 101.745314) (end 117.544 75.719244) (width 0.2) (layer "B.Cu") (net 13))
 (segment (start 122.576628 101.654686) (end 120.595314 103.636) (width 0.2) (layer "B.Cu") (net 13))
 (segment (start 119.434686 103.636) (end 117.544 101.745314) (width 0.2) (layer "B.Cu") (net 13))
 (segment (start 138.484686 103.636) (end 136.503372 101.654686) (width 0.2) (layer "B.Cu") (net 13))
 (segment (start 120.595314 103.636) (end 119.434686 103.636) (width 0.2) (layer "B.Cu") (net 13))
 (segment (start 139.645314 103.636) (end 138.484686 103.636) (width 0.2) (layer "B.Cu") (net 13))
 (segment (start 135.868 62.564) (end 140.466 67.162) (width 0.2) (layer "B.Cu") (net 13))
 (segment (start 136.503372 101.654686) (end 122.576628 101.654686) (width 0.2) (layer "B.Cu") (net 13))
 (segment (start 117.544 75.719244) (end 121.3485 71.914744) (width 0.2) (layer "B.Cu") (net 13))
 (segment (start 140.466 102.815314) (end 139.645314 103.636) (width 0.2) (layer "B.Cu") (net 13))
 (segment (start 116.2685 103.99697) (end 116.2685 71.914744) (width 0.2) (layer "B.Cu") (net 14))
 (segment (start 135.868 67.564) (end 134.166 65.862) (width 0.2) (layer "B.Cu") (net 14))
 (segment (start 145.226 84.751184) (end 145.226 97.902686) (width 0.2) (layer "B.Cu") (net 14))
 (segment (start 141.224 54.8049) (end 141.224 80.749184) (width 0.2) (layer "B.Cu") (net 14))
 (segment (start 141.224 80.749184) (end 145.226 84.751184) (width 0.2) (layer "B.Cu") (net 14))
 (segment (start 134.166 52.7189) (end 136.4859 50.399) (width 0.2) (layer "B.Cu") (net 14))
 (segment (start 141.901184 101.227502) (end 141.901184 102.424) (width 0.2) (layer "B.Cu") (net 14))
 (segment (start 136.4859 50.399) (end 136.8181 50.399) (width 0.2) (layer "B.Cu") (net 14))
 (segment (start 134.166 65.862) (end 134.166 52.7189) (width 0.2) (layer "B.Cu") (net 14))
 (segment (start 141.901184 102.424) (end 137.199184 107.126) (width 0.2) (layer "B.Cu") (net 14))
 (segment (start 145.226 97.902686) (end 141.901184 101.227502) (width 0.2) (layer "B.Cu") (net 14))
 (segment (start 136.8181 50.399) (end 141.224 54.8049) (width 0.2) (layer "B.Cu") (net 14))
 (segment (start 137.199184 107.126) (end 119.39753 107.126) (width 0.2) (layer "B.Cu") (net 14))
 (segment (start 119.39753 107.126) (end 116.2685 103.99697) (width 0.2) (layer "B.Cu") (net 14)))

